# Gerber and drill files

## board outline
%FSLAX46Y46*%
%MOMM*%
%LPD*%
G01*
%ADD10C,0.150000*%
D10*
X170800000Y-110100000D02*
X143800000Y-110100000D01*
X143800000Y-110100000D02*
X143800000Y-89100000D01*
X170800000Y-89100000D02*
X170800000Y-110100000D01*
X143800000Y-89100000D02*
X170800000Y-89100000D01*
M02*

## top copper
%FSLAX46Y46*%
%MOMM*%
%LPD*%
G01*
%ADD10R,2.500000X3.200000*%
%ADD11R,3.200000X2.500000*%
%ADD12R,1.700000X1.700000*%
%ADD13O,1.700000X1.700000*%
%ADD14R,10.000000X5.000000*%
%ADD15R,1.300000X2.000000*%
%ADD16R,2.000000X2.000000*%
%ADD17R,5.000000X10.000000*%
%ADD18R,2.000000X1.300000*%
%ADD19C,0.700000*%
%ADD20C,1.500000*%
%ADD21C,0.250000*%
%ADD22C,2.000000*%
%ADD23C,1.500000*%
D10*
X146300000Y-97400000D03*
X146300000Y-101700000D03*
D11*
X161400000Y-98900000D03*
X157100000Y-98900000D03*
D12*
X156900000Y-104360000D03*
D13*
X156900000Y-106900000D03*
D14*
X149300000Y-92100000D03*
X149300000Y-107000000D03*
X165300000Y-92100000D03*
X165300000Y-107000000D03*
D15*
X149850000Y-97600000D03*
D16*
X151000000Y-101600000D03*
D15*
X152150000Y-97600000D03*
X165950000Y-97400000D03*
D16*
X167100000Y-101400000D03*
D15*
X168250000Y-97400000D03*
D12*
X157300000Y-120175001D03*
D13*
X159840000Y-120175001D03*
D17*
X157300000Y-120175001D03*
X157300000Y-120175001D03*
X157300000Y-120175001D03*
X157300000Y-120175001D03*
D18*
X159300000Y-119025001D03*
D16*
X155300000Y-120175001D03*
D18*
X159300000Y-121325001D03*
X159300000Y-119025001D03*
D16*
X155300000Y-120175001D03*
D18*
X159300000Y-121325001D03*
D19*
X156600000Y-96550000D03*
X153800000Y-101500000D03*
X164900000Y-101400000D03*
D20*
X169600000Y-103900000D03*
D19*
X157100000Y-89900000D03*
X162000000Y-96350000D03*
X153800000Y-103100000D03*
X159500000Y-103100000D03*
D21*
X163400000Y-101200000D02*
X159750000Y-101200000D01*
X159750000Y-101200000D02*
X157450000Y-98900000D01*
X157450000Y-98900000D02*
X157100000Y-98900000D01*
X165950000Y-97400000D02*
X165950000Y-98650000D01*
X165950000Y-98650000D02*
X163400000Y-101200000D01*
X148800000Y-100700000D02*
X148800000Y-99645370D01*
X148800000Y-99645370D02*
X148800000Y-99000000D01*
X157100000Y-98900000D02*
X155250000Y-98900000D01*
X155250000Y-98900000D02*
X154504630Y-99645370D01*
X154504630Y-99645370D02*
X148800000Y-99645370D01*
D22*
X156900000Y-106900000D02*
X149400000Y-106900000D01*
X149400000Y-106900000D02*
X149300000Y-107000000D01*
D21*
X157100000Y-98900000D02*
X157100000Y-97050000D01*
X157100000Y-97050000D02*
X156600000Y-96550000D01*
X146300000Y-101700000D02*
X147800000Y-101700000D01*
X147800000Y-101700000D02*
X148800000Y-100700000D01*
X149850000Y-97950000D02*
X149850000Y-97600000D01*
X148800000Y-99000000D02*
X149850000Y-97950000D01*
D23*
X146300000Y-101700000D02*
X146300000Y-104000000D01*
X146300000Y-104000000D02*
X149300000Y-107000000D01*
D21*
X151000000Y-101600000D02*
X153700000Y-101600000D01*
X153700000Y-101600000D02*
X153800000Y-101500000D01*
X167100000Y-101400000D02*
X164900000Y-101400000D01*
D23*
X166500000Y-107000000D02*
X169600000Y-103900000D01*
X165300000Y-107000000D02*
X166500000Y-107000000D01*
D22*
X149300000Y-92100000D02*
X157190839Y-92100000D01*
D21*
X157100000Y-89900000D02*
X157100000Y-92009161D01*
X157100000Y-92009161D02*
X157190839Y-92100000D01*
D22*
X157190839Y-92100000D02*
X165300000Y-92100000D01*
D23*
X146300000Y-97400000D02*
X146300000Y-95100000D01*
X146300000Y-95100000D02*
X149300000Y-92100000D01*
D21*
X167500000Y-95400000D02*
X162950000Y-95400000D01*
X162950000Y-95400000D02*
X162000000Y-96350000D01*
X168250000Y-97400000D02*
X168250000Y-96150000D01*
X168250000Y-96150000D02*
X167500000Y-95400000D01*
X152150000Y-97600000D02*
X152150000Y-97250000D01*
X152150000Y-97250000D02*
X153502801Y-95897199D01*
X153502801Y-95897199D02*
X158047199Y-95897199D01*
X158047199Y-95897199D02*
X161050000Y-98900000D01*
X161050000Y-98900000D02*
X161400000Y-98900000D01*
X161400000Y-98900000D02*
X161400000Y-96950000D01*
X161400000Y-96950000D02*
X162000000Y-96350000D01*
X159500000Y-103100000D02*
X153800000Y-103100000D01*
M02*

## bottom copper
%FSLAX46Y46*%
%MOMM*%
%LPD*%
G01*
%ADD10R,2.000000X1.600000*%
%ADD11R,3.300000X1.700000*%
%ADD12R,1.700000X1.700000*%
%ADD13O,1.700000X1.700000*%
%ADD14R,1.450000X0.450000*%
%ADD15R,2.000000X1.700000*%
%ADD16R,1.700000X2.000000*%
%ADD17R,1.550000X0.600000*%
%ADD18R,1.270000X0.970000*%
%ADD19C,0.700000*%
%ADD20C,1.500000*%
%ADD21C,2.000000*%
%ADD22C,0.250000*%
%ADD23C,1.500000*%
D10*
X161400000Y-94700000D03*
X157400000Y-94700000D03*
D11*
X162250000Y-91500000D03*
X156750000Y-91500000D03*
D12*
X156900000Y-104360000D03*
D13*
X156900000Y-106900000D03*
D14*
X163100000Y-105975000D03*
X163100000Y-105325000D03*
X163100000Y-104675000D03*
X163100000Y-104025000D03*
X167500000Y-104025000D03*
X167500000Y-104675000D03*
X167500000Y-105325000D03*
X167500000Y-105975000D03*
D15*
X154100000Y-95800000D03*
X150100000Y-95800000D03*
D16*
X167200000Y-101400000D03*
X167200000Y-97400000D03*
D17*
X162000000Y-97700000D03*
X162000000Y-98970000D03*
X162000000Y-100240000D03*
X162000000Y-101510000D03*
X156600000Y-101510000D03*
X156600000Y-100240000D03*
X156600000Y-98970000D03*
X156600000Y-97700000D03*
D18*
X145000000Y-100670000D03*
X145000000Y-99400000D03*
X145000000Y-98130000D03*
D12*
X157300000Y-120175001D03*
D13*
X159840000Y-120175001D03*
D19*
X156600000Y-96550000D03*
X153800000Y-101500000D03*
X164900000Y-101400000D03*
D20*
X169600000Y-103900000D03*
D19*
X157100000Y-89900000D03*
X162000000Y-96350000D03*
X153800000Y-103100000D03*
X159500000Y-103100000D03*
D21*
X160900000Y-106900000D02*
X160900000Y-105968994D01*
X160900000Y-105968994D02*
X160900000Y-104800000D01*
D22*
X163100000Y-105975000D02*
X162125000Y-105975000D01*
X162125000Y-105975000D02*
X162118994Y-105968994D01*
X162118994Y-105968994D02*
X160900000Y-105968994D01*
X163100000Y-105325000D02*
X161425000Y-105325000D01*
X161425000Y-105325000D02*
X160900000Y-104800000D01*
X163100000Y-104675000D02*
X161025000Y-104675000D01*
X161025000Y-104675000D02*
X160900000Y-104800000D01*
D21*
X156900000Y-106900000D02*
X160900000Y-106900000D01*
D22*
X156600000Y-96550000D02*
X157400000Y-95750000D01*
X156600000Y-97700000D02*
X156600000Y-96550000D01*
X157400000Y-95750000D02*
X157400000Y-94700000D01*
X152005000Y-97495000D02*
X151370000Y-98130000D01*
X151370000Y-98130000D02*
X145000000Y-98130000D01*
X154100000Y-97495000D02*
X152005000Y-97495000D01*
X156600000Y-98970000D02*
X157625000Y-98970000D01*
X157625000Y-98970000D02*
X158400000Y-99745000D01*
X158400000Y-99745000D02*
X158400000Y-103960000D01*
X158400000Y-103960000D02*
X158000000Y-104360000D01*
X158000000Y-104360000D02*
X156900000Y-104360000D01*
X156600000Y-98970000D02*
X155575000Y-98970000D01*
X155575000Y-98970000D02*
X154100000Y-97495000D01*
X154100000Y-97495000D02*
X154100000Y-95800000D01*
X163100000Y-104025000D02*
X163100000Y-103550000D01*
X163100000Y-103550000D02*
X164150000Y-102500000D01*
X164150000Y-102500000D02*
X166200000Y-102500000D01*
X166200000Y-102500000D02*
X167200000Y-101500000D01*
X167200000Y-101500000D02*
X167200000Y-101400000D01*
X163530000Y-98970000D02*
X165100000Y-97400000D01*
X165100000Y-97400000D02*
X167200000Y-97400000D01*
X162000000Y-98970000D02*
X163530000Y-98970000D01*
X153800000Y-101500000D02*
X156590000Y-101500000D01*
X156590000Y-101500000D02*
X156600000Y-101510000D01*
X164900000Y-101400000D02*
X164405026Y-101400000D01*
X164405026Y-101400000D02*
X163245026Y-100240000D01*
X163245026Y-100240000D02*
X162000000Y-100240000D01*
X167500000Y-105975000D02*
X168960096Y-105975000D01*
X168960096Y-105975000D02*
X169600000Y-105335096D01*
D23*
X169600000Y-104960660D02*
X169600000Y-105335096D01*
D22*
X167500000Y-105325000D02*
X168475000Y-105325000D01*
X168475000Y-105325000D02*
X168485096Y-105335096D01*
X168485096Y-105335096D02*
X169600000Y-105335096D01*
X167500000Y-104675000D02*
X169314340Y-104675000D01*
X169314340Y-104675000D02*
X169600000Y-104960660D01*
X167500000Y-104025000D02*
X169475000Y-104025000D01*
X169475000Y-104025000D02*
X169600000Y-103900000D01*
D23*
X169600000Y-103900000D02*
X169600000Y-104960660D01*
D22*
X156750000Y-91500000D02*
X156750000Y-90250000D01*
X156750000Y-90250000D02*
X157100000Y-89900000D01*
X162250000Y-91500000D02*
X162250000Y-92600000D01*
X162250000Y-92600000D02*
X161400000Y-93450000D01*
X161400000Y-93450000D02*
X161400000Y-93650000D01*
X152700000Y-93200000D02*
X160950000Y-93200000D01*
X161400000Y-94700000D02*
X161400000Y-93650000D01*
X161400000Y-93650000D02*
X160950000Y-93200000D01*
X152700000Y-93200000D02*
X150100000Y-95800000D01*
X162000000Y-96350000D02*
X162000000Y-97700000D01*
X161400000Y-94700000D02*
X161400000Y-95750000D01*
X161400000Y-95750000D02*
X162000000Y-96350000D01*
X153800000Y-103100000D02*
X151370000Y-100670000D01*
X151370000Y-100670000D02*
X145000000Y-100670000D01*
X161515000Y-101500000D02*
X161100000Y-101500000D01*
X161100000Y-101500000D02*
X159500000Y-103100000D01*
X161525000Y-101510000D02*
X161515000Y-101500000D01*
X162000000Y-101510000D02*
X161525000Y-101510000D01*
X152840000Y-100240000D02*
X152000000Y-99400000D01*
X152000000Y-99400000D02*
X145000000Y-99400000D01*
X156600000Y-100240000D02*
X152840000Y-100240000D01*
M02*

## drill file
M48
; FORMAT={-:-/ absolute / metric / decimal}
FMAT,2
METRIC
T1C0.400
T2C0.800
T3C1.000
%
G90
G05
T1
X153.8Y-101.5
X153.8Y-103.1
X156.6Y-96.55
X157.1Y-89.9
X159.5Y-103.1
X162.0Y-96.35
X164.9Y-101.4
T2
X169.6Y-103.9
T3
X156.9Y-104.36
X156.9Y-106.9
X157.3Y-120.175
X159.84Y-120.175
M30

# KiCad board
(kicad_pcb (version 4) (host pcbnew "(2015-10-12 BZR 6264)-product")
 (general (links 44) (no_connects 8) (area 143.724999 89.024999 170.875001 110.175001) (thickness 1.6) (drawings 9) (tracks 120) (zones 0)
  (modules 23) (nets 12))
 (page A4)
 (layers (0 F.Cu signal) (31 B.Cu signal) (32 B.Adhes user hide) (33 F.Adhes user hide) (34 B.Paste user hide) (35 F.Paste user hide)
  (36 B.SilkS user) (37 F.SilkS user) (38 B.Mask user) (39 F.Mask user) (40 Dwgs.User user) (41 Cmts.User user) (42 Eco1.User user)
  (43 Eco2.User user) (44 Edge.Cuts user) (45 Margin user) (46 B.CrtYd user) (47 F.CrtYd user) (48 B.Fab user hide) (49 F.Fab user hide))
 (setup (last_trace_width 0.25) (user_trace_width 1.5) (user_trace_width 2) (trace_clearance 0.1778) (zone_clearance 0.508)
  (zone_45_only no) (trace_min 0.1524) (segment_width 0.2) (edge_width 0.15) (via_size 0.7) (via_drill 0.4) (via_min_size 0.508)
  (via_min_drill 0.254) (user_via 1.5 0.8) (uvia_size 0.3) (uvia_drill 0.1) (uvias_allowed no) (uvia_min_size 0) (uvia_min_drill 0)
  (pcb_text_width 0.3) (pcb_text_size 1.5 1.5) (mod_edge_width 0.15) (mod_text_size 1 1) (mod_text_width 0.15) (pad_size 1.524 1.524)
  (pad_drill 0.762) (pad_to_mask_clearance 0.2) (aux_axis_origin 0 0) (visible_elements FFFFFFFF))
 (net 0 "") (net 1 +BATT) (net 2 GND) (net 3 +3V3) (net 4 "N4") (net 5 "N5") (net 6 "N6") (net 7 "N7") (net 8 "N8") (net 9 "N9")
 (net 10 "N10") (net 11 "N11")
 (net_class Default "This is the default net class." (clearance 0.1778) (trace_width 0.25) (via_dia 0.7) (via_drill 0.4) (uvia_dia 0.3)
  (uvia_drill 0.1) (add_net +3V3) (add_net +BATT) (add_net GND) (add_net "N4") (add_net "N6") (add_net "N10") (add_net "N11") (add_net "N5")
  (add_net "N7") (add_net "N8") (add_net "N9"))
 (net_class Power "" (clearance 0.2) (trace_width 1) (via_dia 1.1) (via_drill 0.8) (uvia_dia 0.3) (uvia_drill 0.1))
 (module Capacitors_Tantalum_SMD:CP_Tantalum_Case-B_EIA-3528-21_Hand (layer F.Cu) (at 146.3 99.55 270)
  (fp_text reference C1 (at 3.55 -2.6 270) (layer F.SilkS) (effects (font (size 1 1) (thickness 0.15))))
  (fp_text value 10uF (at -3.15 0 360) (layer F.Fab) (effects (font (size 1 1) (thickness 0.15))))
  (pad 1 smd rect (at -2.15 0 270) (size 3.2 2.5) (layers F.Cu F.Paste F.Mask) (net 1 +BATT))
  (pad 2 smd rect (at 2.15 0 270) (size 3.2 2.5) (layers F.Cu F.Paste F.Mask) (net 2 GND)))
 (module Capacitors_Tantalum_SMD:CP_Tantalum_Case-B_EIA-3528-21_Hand (layer F.Cu) (at 159.25 98.9 180)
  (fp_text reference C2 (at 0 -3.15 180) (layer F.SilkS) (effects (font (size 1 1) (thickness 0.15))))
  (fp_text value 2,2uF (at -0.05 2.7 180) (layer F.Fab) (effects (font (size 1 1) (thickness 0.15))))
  (pad 1 smd rect (at -2.15 0 180) (size 3.2 2.5) (layers F.Cu F.Paste F.Mask) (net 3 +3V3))
  (pad 2 smd rect (at 2.15 0 180) (size 3.2 2.5) (layers F.Cu F.Paste F.Mask) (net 2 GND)))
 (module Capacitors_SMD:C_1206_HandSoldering (layer B.Cu) (at 159.4 94.7 180)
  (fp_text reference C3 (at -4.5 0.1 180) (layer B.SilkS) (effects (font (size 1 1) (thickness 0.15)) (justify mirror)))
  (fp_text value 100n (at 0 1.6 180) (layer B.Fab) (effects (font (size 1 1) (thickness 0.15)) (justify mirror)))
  (pad 1 smd rect (at -2 0 180) (size 2 1.6) (layers B.Cu B.Paste B.Mask) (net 3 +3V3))
  (pad 2 smd rect (at 2 0 180) (size 2 1.6) (layers B.Cu B.Paste B.Mask) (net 2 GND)))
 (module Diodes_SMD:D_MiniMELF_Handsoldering (layer B.Cu) (at 159.5 91.5 180)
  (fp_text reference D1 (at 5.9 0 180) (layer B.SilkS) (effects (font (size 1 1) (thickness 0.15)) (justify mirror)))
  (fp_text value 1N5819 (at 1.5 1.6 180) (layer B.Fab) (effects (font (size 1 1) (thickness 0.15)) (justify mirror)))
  (pad 1 smd rect (at -2.75 0 180) (size 3.3 1.7) (layers B.Cu B.Paste B.Mask) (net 3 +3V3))
  (pad 2 smd rect (at 2.75 0 180) (size 3.3 1.7) (layers B.Cu B.Paste B.Mask) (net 1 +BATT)))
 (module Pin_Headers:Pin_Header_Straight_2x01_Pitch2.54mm (layer F.Cu) (at 156.9 104.36 270)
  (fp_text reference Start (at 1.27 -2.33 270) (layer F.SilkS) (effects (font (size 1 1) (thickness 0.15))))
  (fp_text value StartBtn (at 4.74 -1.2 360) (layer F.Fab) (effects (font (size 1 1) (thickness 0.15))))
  (pad 1 thru_hole rect (at 0 0 270) (size 1.7 1.7) (drill 1) (layers *.Cu *.Mask) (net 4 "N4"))
  (pad 2 thru_hole oval (at 2.54 0 270) (size 1.7 1.7) (drill 1) (layers *.Cu *.Mask) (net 2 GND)))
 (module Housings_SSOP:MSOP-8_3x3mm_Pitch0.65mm (layer B.Cu) (at 165.3 105)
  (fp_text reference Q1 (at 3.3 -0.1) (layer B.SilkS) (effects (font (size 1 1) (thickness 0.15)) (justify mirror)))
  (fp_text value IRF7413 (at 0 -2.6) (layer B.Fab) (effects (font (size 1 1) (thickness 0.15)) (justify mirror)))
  (pad 1 smd rect (at -2.2 0.975) (size 1.45 0.45) (layers B.Cu B.Paste B.Mask) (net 2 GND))
  (pad 2 smd rect (at -2.2 0.325) (size 1.45 0.45) (layers B.Cu B.Paste B.Mask) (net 2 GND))
  (pad 3 smd rect (at -2.2 -0.325) (size 1.45 0.45) (layers B.Cu B.Paste B.Mask) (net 2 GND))
  (pad 4 smd rect (at -2.2 -0.975) (size 1.45 0.45) (layers B.Cu B.Paste B.Mask) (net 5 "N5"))
  (pad 5 smd rect (at 2.2 -0.975) (size 1.45 0.45) (layers B.Cu B.Paste B.Mask) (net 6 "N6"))
  (pad 6 smd rect (at 2.2 -0.325) (size 1.45 0.45) (layers B.Cu B.Paste B.Mask) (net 6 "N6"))
  (pad 7 smd rect (at 2.2 0.325) (size 1.45 0.45) (layers B.Cu B.Paste B.Mask) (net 6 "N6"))
  (pad 8 smd rect (at 2.2 0.975) (size 1.45 0.45) (layers B.Cu B.Paste B.Mask) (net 6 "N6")))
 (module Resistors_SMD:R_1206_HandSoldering (layer B.Cu) (at 152.1 95.8 180)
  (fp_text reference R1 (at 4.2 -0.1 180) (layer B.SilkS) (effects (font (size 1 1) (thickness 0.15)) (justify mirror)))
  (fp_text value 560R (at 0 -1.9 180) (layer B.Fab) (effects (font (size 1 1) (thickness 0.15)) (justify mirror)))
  (pad 1 smd rect (at -2 0 180) (size 2 1.7) (layers B.Cu B.Paste B.Mask) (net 4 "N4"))
  (pad 2 smd rect (at 2 0 180) (size 2 1.7) (layers B.Cu B.Paste B.Mask) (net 3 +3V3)))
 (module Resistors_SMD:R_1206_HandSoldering (layer B.Cu) (at 167.2 99.4 90)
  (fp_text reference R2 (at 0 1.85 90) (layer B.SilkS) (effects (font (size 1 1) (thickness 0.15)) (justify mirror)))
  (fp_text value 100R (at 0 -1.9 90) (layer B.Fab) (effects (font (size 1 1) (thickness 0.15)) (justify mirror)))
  (pad 1 smd rect (at -2 0 90) (size 2 1.7) (layers B.Cu B.Paste B.Mask) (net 5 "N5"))
  (pad 2 smd rect (at 2 0 90) (size 2 1.7) (layers B.Cu B.Paste B.Mask) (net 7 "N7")))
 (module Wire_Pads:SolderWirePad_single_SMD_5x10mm (layer F.Cu) (at 149.3 92.1 270)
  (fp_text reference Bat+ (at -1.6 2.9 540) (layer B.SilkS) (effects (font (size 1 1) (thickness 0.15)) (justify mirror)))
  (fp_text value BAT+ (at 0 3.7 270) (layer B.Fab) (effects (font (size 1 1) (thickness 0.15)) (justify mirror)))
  (pad 1 smd rect (at 0 0 270) (size 5 10) (layers F.Cu F.Paste F.Mask) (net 1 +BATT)))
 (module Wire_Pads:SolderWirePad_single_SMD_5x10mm (layer F.Cu) (at 149.3 107 270)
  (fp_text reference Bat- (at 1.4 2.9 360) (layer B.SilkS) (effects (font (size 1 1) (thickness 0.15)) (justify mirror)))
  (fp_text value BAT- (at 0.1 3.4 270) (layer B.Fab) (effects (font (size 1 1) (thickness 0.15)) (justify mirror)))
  (pad 1 smd rect (at 0 0 270) (size 5 10) (layers F.Cu F.Paste F.Mask) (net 2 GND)))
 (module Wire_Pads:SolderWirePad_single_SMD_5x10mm (layer F.Cu) (at 165.3 92.1 90)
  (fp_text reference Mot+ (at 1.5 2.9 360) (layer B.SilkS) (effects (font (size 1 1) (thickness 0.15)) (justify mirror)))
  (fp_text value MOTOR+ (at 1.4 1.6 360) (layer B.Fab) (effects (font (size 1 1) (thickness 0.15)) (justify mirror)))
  (pad 1 smd rect (at 0 0 90) (size 5 10) (layers F.Cu F.Paste F.Mask) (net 1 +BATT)))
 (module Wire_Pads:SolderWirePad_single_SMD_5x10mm (layer F.Cu) (at 165.3 107 90)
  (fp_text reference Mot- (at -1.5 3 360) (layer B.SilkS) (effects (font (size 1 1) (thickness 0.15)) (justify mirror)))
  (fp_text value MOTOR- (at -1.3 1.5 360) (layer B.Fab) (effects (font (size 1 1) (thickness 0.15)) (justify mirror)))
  (pad 1 smd rect (at 0 0 90) (size 5 10) (layers F.Cu F.Paste F.Mask) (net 6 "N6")))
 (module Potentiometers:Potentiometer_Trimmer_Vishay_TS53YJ (layer F.Cu) (at 151 99.6 90)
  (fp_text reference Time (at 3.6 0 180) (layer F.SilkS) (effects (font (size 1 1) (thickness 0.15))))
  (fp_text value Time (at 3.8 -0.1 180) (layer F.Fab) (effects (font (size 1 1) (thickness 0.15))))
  (pad 1 smd rect (at 2 -1.15 90) (size 2 1.3) (layers F.Cu F.Mask) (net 2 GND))
  (pad 2 smd rect (at -2 0 90) (size 2 2) (layers F.Cu F.Mask) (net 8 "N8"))
  (pad 3 smd rect (at 2 1.15 90) (size 2 1.3) (layers F.Cu F.Mask) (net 3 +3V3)))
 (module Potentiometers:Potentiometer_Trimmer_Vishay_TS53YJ (layer F.Cu) (at 167.1 99.4 90)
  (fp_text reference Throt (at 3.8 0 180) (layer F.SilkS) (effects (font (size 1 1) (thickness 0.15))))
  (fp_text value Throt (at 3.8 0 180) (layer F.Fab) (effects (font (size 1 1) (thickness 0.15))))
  (pad 1 smd rect (at 2 -1.15 90) (size 2 1.3) (layers F.Cu F.Mask) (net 2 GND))
  (pad 2 smd rect (at -2 0 90) (size 2 2) (layers F.Cu F.Mask) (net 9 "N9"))
  (pad 3 smd rect (at 2 1.15 90) (size 2 1.3) (layers F.Cu F.Mask) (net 3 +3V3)))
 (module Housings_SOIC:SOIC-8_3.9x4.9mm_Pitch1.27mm (layer B.Cu) (at 159.3 99.605 180)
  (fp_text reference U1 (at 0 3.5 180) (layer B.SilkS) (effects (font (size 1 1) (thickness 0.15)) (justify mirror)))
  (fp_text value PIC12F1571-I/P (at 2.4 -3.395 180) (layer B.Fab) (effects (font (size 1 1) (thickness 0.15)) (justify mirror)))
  (pad 1 smd rect (at -2.7 1.905 180) (size 1.55 0.6) (layers B.Cu B.Paste B.Mask) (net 3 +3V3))
  (pad 2 smd rect (at -2.7 0.635 180) (size 1.55 0.6) (layers B.Cu B.Paste B.Mask) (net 7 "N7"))
  (pad 3 smd rect (at -2.7 -0.635 180) (size 1.55 0.6) (layers B.Cu B.Paste B.Mask) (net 9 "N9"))
  (pad 4 smd rect (at -2.7 -1.905 180) (size 1.55 0.6) (layers B.Cu B.Paste B.Mask) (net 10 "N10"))
  (pad 5 smd rect (at 2.7 -1.905 180) (size 1.55 0.6) (layers B.Cu B.Paste B.Mask) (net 8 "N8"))
  (pad 6 smd rect (at 2.7 -0.635 180) (size 1.55 0.6) (layers B.Cu B.Paste B.Mask) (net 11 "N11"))
  (pad 7 smd rect (at 2.7 0.635 180) (size 1.55 0.6) (layers B.Cu B.Paste B.Mask) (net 4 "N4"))
  (pad 8 smd rect (at 2.7 1.905 180) (size 1.55 0.6) (layers B.Cu B.Paste B.Mask) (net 2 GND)))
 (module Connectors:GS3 (layer B.Cu) (at 145 99.4)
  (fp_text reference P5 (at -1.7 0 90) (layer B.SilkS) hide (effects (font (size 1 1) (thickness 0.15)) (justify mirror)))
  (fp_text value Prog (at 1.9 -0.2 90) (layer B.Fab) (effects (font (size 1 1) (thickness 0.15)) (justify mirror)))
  (pad 1 smd rect (at 0 1.27) (size 1.27 0.97) (layers B.Cu B.Paste B.Mask) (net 10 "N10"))
  (pad 2 smd rect (at 0 0) (size 1.27 0.97) (layers B.Cu B.Paste B.Mask) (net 11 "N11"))
  (pad 3 smd rect (at 0 -1.27) (size 1.27 0.97) (layers B.Cu B.Paste B.Mask) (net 4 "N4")))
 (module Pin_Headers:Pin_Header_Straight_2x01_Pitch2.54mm (layer F.Cu) (at 157.3 120.175001)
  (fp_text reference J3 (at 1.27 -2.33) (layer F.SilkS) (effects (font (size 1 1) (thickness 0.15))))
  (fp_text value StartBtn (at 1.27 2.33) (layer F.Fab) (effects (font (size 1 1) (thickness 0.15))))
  (pad 1 thru_hole rect (at 0 0) (size 1.7 1.7) (drill 1) (layers *.Cu *.Mask) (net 4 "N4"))
  (pad 2 thru_hole oval (at 2.54 0) (size 1.7 1.7) (drill 1) (layers *.Cu *.Mask) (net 2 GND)))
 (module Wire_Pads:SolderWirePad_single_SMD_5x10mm (layer F.Cu) (at 157.3 120.175001)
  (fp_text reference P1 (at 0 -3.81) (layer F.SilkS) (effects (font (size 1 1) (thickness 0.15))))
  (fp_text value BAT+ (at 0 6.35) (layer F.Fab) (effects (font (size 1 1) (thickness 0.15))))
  (pad 1 smd rect (at 0 0) (size 5 10) (layers F.Cu F.Paste F.Mask) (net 1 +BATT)))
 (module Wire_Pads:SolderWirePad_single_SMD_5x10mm (layer F.Cu) (at 157.3 120.175001)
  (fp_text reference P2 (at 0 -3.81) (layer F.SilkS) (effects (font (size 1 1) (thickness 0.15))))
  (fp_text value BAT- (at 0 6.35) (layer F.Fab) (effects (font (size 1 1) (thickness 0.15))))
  (pad 1 smd rect (at 0 0) (size 5 10) (layers F.Cu F.Paste F.Mask) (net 2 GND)))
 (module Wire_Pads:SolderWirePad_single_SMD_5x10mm (layer F.Cu) (at 157.3 120.175001)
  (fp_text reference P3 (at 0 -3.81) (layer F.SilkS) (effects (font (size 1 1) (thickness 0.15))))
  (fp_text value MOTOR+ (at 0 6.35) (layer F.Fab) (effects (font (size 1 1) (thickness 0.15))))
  (pad 1 smd rect (at 0 0) (size 5 10) (layers F.Cu F.Paste F.Mask) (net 1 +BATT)))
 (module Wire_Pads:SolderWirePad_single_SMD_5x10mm (layer F.Cu) (at 157.3 120.175001)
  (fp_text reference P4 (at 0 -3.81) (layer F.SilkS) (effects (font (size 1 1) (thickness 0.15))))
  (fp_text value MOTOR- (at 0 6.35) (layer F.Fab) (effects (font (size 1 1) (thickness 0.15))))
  (pad 1 smd rect (at 0 0) (size 5 10) (layers F.Cu F.Paste F.Mask) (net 6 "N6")))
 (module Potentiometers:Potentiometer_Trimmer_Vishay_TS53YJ (layer F.Cu) (at 157.3 120.175001)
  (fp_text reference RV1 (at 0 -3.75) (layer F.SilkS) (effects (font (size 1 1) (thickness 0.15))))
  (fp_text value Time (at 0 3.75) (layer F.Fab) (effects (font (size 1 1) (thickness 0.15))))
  (pad 1 smd rect (at 2 -1.15) (size 2 1.3) (layers F.Cu F.Mask) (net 2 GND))
  (pad 2 smd rect (at -2 0) (size 2 2) (layers F.Cu F.Mask) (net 8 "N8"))
  (pad 3 smd rect (at 2 1.15) (size 2 1.3) (layers F.Cu F.Mask) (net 3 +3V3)))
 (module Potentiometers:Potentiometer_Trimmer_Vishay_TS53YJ (layer F.Cu) (at 157.3 120.175001)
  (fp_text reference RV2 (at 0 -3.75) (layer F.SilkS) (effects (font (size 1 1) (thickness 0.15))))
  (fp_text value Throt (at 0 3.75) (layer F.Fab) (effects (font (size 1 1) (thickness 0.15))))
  (pad 1 smd rect (at 2 -1.15) (size 2 1.3) (layers F.Cu F.Mask) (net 2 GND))
  (pad 2 smd rect (at -2 0) (size 2 2) (layers F.Cu F.Mask) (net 9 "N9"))
  (pad 3 smd rect (at 2 1.15) (size 2 1.3) (layers F.Cu F.Mask) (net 3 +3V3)))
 (gr_line (start 170.8 110.1) (end 143.8 110.1) (angle 90) (layer Edge.Cuts) (width 0.15))
 (gr_line (start 143.8 110.1) (end 143.8 89.1) (angle 90) (layer Edge.Cuts) (width 0.15))
 (gr_line (start 170.8 89.1) (end 170.8 110.1) (angle 90) (layer Edge.Cuts) (width 0.15))
 (gr_line (start 143.8 89.1) (end 170.8 89.1) (angle 90) (layer Edge.Cuts) (width 0.15))
 (segment (start 160.9 106.9) (end 160.9 105.968994) (width 2) (layer B.Cu) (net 2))
 (segment (start 160.9 105.968994) (end 160.9 104.8) (width 2) (layer B.Cu) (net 2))
 (segment (start 163.1 105.975) (end 162.125 105.975) (width 0.25) (layer B.Cu) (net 2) (status 10))
 (segment (start 162.125 105.975) (end 162.118994 105.968994) (width 0.25) (layer B.Cu) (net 2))
 (segment (start 162.118994 105.968994) (end 160.9 105.968994) (width 0.25) (layer B.Cu) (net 2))
 (segment (start 163.1 105.325) (end 161.425 105.325) (width 0.25) (layer B.Cu) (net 2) (status 10))
 (segment (start 161.425 105.325) (end 160.9 104.8) (width 0.25) (layer B.Cu) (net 2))
 (segment (start 163.1 104.675) (end 161.025 104.675) (width 0.25) (layer B.Cu) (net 2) (status 10))
 (segment (start 161.025 104.675) (end 160.9 104.8) (width 0.25) (layer B.Cu) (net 2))
 (segment (start 156.9 106.9) (end 160.9 106.9) (width 2) (layer B.Cu) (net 2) (status 10))
 (segment (start 163.4 101.2) (end 159.75 101.2) (width 0.25) (layer F.Cu) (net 2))
 (segment (start 159.75 101.2) (end 157.45 98.9) (width 0.25) (layer F.Cu) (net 2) (status 20))
 (segment (start 157.45 98.9) (end 157.1 98.9) (width 0.25) (layer F.Cu) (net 2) (status 30))
 (segment (start 165.95 97.4) (end 165.95 98.65) (width 0.25) (layer F.Cu) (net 2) (status 10))
 (segment (start 165.95 98.65) (end 163.4 101.2) (width 0.25) (layer F.Cu) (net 2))
 (segment (start 148.8 100.7) (end 148.8 99.64537) (width 0.25) (layer F.Cu) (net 2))
 (segment (start 148.8 99.64537) (end 148.8 99) (width 0.25) (layer F.Cu) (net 2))
 (segment (start 157.1 98.9) (end 155.25 98.9) (width 0.25) (layer F.Cu) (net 2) (status 10))
 (segment (start 155.25 98.9) (end 154.50463 99.64537) (width 0.25) (layer F.Cu) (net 2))
 (segment (start 154.50463 99.64537) (end 148.8 99.64537) (width 0.25) (layer F.Cu) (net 2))
 (segment (start 156.9 106.9) (end 149.4 106.9) (width 2) (layer F.Cu) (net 2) (status 30))
 (segment (start 149.4 106.9) (end 149.3 107) (width 2) (layer F.Cu) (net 2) (status 30))
 (segment (start 157.1 98.9) (end 157.1 97.05) (width 0.25) (layer F.Cu) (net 2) (status 10))
 (segment (start 157.1 97.05) (end 156.6 96.55) (width 0.25) (layer F.Cu) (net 2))
 (segment (start 156.6 96.55) (end 157.4 95.75) (width 0.25) (layer B.Cu) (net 2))
 (via (at 156.6 96.55) (size 0.7) (drill 0.4) (layers F.Cu B.Cu) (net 2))
 (segment (start 156.6 97.7) (end 156.6 96.55) (width 0.25) (layer B.Cu) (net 2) (status 10))
 (segment (start 157.4 95.75) (end 157.4 94.7) (width 0.25) (layer B.Cu) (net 2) (status 20))
 (segment (start 146.3 101.7) (end 147.8 101.7) (width 0.25) (layer F.Cu) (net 2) (status 10))
 (segment (start 147.8 101.7) (end 148.8 100.7) (width 0.25) (layer F.Cu) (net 2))
 (segment (start 149.85 97.95) (end 149.85 97.6) (width 0.25) (layer F.Cu) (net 2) (status 30))
 (segment (start 148.8 99) (end 149.85 97.95) (width 0.25) (layer F.Cu) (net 2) (status 20))
 (segment (start 146.3 101.7) (end 146.3 104) (width 1.5) (layer F.Cu) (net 2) (status 10))
 (segment (start 146.3 104) (end 149.3 107) (width 1.5) (layer F.Cu) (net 2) (status 20))
 (segment (start 152.005 97.495) (end 151.37 98.13) (width 0.25) (layer B.Cu) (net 4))
 (segment (start 151.37 98.13) (end 145 98.13) (width 0.25) (layer B.Cu) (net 4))
 (segment (start 154.1 97.495) (end 152.005 97.495) (width 0.25) (layer B.Cu) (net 4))
 (segment (start 156.6 98.97) (end 157.625 98.97) (width 0.25) (layer B.Cu) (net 4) (status 10))
 (segment (start 157.625 98.97) (end 158.4 99.745) (width 0.25) (layer B.Cu) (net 4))
 (segment (start 158.4 99.745) (end 158.4 103.96) (width 0.25) (layer B.Cu) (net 4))
 (segment (start 158.4 103.96) (end 158 104.36) (width 0.25) (layer B.Cu) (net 4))
 (segment (start 158 104.36) (end 156.9 104.36) (width 0.25) (layer B.Cu) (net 4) (status 20))
 (segment (start 156.6 98.97) (end 155.575 98.97) (width 0.25) (layer B.Cu) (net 4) (status 10))
 (segment (start 155.575 98.97) (end 154.1 97.495) (width 0.25) (layer B.Cu) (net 4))
 (segment (start 154.1 97.495) (end 154.1 95.8) (width 0.25) (layer B.Cu) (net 4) (status 20))
 (segment (start 163.1 104.025) (end 163.1 103.55) (width 0.25) (layer B.Cu) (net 5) (status 10))
 (segment (start 163.1 103.55) (end 164.15 102.5) (width 0.25) (layer B.Cu) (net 5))
 (segment (start 164.15 102.5) (end 166.2 102.5) (width 0.25) (layer B.Cu) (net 5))
 (segment (start 166.2 102.5) (end 167.2 101.5) (width 0.25) (layer B.Cu) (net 5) (status 20))
 (segment (start 167.2 101.5) (end 167.2 101.4) (width 0.25) (layer B.Cu) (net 5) (status 30))
 (segment (start 163.53 98.97) (end 165.1 97.4) (width 0.25) (layer B.Cu) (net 7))
 (segment (start 165.1 97.4) (end 167.2 97.4) (width 0.25) (layer B.Cu) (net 7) (status 20))
 (segment (start 162 98.97) (end 163.53 98.97) (width 0.25) (layer B.Cu) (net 7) (status 10))
 (segment (start 153.8 101.5) (end 156.59 101.5) (width 0.25) (layer B.Cu) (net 8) (status 20))
 (segment (start 156.59 101.5) (end 156.6 101.51) (width 0.25) (layer B.Cu) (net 8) (status 30))
 (segment (start 151 101.6) (end 153.7 101.6) (width 0.25) (layer F.Cu) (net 8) (status 10))
 (segment (start 153.7 101.6) (end 153.8 101.5) (width 0.25) (layer F.Cu) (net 8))
 (via (at 153.8 101.5) (size 0.7) (drill 0.4) (layers F.Cu B.Cu) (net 8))
 (segment (start 164.9 101.4) (end 164.405026 101.4) (width 0.25) (layer B.Cu) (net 9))
 (segment (start 164.405026 101.4) (end 163.245026 100.24) (width 0.25) (layer B.Cu) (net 9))
 (segment (start 163.245026 100.24) (end 162 100.24) (width 0.25) (layer B.Cu) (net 9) (status 20))
 (segment (start 167.1 101.4) (end 164.9 101.4) (width 0.25) (layer F.Cu) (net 9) (status 10))
 (via (at 164.9 101.4) (size 0.7) (drill 0.4) (layers F.Cu B.Cu) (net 9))
 (segment (start 167.5 105.975) (end 168.960096 105.975) (width 0.25) (layer B.Cu) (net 6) (status 10))
 (segment (start 168.960096 105.975) (end 169.6 105.335096) (width 0.25) (layer B.Cu) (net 6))
 (segment (start 169.6 104.96066) (end 169.6 105.335096) (width 1.5) (layer B.Cu) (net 6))
 (segment (start 167.5 105.325) (end 168.475 105.325) (width 0.25) (layer B.Cu) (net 6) (status 10))
 (segment (start 168.475 105.325) (end 168.485096 105.335096) (width 0.25) (layer B.Cu) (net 6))
 (segment (start 168.485096 105.335096) (end 169.6 105.335096) (width 0.25) (layer B.Cu) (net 6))
 (segment (start 167.5 104.675) (end 169.31434 104.675) (width 0.25) (layer B.Cu) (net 6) (status 10))
 (segment (start 169.31434 104.675) (end 169.6 104.96066) (width 0.25) (layer B.Cu) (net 6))
 (segment (start 167.5 104.025) (end 169.475 104.025) (width 0.25) (layer B.Cu) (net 6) (status 10))
 (segment (start 169.475 104.025) (end 169.6 103.9) (width 0.25) (layer B.Cu) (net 6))
 (segment (start 169.6 103.9) (end 169.6 104.96066) (width 1.5) (layer B.Cu) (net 6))
 (segment (start 166.5 107) (end 169.6 103.9) (width 1.5) (layer F.Cu) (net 6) (status 10))
 (via (at 169.6 103.9) (size 1.5) (drill 0.8) (layers F.Cu B.Cu) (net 6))
 (segment (start 165.3 107) (end 166.5 107) (width 1.5) (layer F.Cu) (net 6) (status 30))
 (segment (start 149.3 92.1) (end 157.190839 92.1) (width 2) (layer F.Cu) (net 1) (status 10))
 (segment (start 157.1 89.9) (end 157.1 92.009161) (width 0.25) (layer F.Cu) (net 1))
 (segment (start 157.1 92.009161) (end 157.190839 92.1) (width 0.25) (layer F.Cu) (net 1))
 (segment (start 157.190839 92.1) (end 165.3 92.1) (width 2) (layer F.Cu) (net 1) (status 20))
 (segment (start 156.75 91.5) (end 156.75 90.25) (width 0.25) (layer B.Cu) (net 1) (status 10))
 (segment (start 156.75 90.25) (end 157.1 89.9) (width 0.25) (layer B.Cu) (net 1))
 (via (at 157.1 89.9) (size 0.7) (drill 0.4) (layers F.Cu B.Cu) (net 1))
 (segment (start 146.3 97.4) (end 146.3 95.1) (width 1.5) (layer F.Cu) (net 1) (status 10))
 (segment (start 146.3 95.1) (end 149.3 92.1) (width 1.5) (layer F.Cu) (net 1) (status 20))
 (segment (start 167.5 95.4) (end 162.95 95.4) (width 0.25) (layer F.Cu) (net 3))
 (segment (start 162.95 95.4) (end 162 96.35) (width 0.25) (layer F.Cu) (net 3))
 (segment (start 168.25 97.4) (end 168.25 96.15) (width 0.25) (layer F.Cu) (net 3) (status 10))
 (segment (start 168.25 96.15) (end 167.5 95.4) (width 0.25) (layer F.Cu) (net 3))
 (segment (start 162.25 91.5) (end 162.25 92.6) (width 0.25) (layer B.Cu) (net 3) (status 10))
 (segment (start 162.25 92.6) (end 161.4 93.45) (width 0.25) (layer B.Cu) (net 3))
 (segment (start 161.4 93.45) (end 161.4 93.65) (width 0.25) (layer B.Cu) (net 3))
 (segment (start 152.7 93.2) (end 160.95 93.2) (width 0.25) (layer B.Cu) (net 3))
 (segment (start 161.4 94.7) (end 161.4 93.65) (width 0.25) (layer B.Cu) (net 3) (status 10))
 (segment (start 161.4 93.65) (end 160.95 93.2) (width 0.25) (layer B.Cu) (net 3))
 (segment (start 152.7 93.2) (end 150.1 95.8) (width 0.25) (layer B.Cu) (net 3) (status 20))
 (segment (start 152.15 97.6) (end 152.15 97.25) (width 0.25) (layer F.Cu) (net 3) (status 30))
 (segment (start 152.15 97.25) (end 153.502801 95.897199) (width 0.25) (layer F.Cu) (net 3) (status 10))
 (segment (start 153.502801 95.897199) (end 158.047199 95.897199) (width 0.25) (layer F.Cu) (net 3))
 (segment (start 158.047199 95.897199) (end 161.05 98.9) (width 0.25) (layer F.Cu) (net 3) (status 20))
 (segment (start 161.05 98.9) (end 161.4 98.9) (width 0.25) (layer F.Cu) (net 3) (status 30))
 (segment (start 161.4 98.9) (end 161.4 96.95) (width 0.25) (layer F.Cu) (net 3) (status 10))
 (segment (start 161.4 96.95) (end 162 96.35) (width 0.25) (layer F.Cu) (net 3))
 (via (at 162 96.35) (size 0.7) (drill 0.4) (layers F.Cu B.Cu) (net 3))
 (segment (start 162 96.35) (end 162 97.7) (width 0.25) (layer B.Cu) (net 3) (status 20))
 (segment (start 161.4 94.7) (end 161.4 95.75) (width 0.25) (layer B.Cu) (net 3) (status 10))
 (segment (start 161.4 95.75) (end 162 96.35) (width 0.25) (layer B.Cu) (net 3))
 (segment (start 153.8 103.1) (end 151.37 100.67) (width 0.25) (layer B.Cu) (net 10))
 (segment (start 151.37 100.67) (end 145 100.67) (width 0.25) (layer B.Cu) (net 10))
 (segment (start 159.5 103.1) (end 153.8 103.1) (width 0.25) (layer F.Cu) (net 10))
 (via (at 153.8 103.1) (size 0.7) (drill 0.4) (layers F.Cu B.Cu) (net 10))
 (segment (start 161.515 101.5) (end 161.1 101.5) (width 0.25) (layer B.Cu) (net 10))
 (segment (start 161.1 101.5) (end 159.5 103.1) (width 0.25) (layer B.Cu) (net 10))
 (via (at 159.5 103.1) (size 0.7) (drill 0.4) (layers F.Cu B.Cu) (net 10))
 (segment (start 161.525 101.51) (end 161.515 101.5) (width 0.25) (layer B.Cu) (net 10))
 (segment (start 162 101.51) (end 161.525 101.51) (width 0.25) (layer B.Cu) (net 10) (status 30))
 (segment (start 152.84 100.24) (end 152 99.4) (width 0.25) (layer B.Cu) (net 11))
 (segment (start 152 99.4) (end 145 99.4) (width 0.25) (layer B.Cu) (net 11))
 (segment (start 156.6 100.24) (end 152.84 100.24) (width 0.25) (layer B.Cu) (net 11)))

